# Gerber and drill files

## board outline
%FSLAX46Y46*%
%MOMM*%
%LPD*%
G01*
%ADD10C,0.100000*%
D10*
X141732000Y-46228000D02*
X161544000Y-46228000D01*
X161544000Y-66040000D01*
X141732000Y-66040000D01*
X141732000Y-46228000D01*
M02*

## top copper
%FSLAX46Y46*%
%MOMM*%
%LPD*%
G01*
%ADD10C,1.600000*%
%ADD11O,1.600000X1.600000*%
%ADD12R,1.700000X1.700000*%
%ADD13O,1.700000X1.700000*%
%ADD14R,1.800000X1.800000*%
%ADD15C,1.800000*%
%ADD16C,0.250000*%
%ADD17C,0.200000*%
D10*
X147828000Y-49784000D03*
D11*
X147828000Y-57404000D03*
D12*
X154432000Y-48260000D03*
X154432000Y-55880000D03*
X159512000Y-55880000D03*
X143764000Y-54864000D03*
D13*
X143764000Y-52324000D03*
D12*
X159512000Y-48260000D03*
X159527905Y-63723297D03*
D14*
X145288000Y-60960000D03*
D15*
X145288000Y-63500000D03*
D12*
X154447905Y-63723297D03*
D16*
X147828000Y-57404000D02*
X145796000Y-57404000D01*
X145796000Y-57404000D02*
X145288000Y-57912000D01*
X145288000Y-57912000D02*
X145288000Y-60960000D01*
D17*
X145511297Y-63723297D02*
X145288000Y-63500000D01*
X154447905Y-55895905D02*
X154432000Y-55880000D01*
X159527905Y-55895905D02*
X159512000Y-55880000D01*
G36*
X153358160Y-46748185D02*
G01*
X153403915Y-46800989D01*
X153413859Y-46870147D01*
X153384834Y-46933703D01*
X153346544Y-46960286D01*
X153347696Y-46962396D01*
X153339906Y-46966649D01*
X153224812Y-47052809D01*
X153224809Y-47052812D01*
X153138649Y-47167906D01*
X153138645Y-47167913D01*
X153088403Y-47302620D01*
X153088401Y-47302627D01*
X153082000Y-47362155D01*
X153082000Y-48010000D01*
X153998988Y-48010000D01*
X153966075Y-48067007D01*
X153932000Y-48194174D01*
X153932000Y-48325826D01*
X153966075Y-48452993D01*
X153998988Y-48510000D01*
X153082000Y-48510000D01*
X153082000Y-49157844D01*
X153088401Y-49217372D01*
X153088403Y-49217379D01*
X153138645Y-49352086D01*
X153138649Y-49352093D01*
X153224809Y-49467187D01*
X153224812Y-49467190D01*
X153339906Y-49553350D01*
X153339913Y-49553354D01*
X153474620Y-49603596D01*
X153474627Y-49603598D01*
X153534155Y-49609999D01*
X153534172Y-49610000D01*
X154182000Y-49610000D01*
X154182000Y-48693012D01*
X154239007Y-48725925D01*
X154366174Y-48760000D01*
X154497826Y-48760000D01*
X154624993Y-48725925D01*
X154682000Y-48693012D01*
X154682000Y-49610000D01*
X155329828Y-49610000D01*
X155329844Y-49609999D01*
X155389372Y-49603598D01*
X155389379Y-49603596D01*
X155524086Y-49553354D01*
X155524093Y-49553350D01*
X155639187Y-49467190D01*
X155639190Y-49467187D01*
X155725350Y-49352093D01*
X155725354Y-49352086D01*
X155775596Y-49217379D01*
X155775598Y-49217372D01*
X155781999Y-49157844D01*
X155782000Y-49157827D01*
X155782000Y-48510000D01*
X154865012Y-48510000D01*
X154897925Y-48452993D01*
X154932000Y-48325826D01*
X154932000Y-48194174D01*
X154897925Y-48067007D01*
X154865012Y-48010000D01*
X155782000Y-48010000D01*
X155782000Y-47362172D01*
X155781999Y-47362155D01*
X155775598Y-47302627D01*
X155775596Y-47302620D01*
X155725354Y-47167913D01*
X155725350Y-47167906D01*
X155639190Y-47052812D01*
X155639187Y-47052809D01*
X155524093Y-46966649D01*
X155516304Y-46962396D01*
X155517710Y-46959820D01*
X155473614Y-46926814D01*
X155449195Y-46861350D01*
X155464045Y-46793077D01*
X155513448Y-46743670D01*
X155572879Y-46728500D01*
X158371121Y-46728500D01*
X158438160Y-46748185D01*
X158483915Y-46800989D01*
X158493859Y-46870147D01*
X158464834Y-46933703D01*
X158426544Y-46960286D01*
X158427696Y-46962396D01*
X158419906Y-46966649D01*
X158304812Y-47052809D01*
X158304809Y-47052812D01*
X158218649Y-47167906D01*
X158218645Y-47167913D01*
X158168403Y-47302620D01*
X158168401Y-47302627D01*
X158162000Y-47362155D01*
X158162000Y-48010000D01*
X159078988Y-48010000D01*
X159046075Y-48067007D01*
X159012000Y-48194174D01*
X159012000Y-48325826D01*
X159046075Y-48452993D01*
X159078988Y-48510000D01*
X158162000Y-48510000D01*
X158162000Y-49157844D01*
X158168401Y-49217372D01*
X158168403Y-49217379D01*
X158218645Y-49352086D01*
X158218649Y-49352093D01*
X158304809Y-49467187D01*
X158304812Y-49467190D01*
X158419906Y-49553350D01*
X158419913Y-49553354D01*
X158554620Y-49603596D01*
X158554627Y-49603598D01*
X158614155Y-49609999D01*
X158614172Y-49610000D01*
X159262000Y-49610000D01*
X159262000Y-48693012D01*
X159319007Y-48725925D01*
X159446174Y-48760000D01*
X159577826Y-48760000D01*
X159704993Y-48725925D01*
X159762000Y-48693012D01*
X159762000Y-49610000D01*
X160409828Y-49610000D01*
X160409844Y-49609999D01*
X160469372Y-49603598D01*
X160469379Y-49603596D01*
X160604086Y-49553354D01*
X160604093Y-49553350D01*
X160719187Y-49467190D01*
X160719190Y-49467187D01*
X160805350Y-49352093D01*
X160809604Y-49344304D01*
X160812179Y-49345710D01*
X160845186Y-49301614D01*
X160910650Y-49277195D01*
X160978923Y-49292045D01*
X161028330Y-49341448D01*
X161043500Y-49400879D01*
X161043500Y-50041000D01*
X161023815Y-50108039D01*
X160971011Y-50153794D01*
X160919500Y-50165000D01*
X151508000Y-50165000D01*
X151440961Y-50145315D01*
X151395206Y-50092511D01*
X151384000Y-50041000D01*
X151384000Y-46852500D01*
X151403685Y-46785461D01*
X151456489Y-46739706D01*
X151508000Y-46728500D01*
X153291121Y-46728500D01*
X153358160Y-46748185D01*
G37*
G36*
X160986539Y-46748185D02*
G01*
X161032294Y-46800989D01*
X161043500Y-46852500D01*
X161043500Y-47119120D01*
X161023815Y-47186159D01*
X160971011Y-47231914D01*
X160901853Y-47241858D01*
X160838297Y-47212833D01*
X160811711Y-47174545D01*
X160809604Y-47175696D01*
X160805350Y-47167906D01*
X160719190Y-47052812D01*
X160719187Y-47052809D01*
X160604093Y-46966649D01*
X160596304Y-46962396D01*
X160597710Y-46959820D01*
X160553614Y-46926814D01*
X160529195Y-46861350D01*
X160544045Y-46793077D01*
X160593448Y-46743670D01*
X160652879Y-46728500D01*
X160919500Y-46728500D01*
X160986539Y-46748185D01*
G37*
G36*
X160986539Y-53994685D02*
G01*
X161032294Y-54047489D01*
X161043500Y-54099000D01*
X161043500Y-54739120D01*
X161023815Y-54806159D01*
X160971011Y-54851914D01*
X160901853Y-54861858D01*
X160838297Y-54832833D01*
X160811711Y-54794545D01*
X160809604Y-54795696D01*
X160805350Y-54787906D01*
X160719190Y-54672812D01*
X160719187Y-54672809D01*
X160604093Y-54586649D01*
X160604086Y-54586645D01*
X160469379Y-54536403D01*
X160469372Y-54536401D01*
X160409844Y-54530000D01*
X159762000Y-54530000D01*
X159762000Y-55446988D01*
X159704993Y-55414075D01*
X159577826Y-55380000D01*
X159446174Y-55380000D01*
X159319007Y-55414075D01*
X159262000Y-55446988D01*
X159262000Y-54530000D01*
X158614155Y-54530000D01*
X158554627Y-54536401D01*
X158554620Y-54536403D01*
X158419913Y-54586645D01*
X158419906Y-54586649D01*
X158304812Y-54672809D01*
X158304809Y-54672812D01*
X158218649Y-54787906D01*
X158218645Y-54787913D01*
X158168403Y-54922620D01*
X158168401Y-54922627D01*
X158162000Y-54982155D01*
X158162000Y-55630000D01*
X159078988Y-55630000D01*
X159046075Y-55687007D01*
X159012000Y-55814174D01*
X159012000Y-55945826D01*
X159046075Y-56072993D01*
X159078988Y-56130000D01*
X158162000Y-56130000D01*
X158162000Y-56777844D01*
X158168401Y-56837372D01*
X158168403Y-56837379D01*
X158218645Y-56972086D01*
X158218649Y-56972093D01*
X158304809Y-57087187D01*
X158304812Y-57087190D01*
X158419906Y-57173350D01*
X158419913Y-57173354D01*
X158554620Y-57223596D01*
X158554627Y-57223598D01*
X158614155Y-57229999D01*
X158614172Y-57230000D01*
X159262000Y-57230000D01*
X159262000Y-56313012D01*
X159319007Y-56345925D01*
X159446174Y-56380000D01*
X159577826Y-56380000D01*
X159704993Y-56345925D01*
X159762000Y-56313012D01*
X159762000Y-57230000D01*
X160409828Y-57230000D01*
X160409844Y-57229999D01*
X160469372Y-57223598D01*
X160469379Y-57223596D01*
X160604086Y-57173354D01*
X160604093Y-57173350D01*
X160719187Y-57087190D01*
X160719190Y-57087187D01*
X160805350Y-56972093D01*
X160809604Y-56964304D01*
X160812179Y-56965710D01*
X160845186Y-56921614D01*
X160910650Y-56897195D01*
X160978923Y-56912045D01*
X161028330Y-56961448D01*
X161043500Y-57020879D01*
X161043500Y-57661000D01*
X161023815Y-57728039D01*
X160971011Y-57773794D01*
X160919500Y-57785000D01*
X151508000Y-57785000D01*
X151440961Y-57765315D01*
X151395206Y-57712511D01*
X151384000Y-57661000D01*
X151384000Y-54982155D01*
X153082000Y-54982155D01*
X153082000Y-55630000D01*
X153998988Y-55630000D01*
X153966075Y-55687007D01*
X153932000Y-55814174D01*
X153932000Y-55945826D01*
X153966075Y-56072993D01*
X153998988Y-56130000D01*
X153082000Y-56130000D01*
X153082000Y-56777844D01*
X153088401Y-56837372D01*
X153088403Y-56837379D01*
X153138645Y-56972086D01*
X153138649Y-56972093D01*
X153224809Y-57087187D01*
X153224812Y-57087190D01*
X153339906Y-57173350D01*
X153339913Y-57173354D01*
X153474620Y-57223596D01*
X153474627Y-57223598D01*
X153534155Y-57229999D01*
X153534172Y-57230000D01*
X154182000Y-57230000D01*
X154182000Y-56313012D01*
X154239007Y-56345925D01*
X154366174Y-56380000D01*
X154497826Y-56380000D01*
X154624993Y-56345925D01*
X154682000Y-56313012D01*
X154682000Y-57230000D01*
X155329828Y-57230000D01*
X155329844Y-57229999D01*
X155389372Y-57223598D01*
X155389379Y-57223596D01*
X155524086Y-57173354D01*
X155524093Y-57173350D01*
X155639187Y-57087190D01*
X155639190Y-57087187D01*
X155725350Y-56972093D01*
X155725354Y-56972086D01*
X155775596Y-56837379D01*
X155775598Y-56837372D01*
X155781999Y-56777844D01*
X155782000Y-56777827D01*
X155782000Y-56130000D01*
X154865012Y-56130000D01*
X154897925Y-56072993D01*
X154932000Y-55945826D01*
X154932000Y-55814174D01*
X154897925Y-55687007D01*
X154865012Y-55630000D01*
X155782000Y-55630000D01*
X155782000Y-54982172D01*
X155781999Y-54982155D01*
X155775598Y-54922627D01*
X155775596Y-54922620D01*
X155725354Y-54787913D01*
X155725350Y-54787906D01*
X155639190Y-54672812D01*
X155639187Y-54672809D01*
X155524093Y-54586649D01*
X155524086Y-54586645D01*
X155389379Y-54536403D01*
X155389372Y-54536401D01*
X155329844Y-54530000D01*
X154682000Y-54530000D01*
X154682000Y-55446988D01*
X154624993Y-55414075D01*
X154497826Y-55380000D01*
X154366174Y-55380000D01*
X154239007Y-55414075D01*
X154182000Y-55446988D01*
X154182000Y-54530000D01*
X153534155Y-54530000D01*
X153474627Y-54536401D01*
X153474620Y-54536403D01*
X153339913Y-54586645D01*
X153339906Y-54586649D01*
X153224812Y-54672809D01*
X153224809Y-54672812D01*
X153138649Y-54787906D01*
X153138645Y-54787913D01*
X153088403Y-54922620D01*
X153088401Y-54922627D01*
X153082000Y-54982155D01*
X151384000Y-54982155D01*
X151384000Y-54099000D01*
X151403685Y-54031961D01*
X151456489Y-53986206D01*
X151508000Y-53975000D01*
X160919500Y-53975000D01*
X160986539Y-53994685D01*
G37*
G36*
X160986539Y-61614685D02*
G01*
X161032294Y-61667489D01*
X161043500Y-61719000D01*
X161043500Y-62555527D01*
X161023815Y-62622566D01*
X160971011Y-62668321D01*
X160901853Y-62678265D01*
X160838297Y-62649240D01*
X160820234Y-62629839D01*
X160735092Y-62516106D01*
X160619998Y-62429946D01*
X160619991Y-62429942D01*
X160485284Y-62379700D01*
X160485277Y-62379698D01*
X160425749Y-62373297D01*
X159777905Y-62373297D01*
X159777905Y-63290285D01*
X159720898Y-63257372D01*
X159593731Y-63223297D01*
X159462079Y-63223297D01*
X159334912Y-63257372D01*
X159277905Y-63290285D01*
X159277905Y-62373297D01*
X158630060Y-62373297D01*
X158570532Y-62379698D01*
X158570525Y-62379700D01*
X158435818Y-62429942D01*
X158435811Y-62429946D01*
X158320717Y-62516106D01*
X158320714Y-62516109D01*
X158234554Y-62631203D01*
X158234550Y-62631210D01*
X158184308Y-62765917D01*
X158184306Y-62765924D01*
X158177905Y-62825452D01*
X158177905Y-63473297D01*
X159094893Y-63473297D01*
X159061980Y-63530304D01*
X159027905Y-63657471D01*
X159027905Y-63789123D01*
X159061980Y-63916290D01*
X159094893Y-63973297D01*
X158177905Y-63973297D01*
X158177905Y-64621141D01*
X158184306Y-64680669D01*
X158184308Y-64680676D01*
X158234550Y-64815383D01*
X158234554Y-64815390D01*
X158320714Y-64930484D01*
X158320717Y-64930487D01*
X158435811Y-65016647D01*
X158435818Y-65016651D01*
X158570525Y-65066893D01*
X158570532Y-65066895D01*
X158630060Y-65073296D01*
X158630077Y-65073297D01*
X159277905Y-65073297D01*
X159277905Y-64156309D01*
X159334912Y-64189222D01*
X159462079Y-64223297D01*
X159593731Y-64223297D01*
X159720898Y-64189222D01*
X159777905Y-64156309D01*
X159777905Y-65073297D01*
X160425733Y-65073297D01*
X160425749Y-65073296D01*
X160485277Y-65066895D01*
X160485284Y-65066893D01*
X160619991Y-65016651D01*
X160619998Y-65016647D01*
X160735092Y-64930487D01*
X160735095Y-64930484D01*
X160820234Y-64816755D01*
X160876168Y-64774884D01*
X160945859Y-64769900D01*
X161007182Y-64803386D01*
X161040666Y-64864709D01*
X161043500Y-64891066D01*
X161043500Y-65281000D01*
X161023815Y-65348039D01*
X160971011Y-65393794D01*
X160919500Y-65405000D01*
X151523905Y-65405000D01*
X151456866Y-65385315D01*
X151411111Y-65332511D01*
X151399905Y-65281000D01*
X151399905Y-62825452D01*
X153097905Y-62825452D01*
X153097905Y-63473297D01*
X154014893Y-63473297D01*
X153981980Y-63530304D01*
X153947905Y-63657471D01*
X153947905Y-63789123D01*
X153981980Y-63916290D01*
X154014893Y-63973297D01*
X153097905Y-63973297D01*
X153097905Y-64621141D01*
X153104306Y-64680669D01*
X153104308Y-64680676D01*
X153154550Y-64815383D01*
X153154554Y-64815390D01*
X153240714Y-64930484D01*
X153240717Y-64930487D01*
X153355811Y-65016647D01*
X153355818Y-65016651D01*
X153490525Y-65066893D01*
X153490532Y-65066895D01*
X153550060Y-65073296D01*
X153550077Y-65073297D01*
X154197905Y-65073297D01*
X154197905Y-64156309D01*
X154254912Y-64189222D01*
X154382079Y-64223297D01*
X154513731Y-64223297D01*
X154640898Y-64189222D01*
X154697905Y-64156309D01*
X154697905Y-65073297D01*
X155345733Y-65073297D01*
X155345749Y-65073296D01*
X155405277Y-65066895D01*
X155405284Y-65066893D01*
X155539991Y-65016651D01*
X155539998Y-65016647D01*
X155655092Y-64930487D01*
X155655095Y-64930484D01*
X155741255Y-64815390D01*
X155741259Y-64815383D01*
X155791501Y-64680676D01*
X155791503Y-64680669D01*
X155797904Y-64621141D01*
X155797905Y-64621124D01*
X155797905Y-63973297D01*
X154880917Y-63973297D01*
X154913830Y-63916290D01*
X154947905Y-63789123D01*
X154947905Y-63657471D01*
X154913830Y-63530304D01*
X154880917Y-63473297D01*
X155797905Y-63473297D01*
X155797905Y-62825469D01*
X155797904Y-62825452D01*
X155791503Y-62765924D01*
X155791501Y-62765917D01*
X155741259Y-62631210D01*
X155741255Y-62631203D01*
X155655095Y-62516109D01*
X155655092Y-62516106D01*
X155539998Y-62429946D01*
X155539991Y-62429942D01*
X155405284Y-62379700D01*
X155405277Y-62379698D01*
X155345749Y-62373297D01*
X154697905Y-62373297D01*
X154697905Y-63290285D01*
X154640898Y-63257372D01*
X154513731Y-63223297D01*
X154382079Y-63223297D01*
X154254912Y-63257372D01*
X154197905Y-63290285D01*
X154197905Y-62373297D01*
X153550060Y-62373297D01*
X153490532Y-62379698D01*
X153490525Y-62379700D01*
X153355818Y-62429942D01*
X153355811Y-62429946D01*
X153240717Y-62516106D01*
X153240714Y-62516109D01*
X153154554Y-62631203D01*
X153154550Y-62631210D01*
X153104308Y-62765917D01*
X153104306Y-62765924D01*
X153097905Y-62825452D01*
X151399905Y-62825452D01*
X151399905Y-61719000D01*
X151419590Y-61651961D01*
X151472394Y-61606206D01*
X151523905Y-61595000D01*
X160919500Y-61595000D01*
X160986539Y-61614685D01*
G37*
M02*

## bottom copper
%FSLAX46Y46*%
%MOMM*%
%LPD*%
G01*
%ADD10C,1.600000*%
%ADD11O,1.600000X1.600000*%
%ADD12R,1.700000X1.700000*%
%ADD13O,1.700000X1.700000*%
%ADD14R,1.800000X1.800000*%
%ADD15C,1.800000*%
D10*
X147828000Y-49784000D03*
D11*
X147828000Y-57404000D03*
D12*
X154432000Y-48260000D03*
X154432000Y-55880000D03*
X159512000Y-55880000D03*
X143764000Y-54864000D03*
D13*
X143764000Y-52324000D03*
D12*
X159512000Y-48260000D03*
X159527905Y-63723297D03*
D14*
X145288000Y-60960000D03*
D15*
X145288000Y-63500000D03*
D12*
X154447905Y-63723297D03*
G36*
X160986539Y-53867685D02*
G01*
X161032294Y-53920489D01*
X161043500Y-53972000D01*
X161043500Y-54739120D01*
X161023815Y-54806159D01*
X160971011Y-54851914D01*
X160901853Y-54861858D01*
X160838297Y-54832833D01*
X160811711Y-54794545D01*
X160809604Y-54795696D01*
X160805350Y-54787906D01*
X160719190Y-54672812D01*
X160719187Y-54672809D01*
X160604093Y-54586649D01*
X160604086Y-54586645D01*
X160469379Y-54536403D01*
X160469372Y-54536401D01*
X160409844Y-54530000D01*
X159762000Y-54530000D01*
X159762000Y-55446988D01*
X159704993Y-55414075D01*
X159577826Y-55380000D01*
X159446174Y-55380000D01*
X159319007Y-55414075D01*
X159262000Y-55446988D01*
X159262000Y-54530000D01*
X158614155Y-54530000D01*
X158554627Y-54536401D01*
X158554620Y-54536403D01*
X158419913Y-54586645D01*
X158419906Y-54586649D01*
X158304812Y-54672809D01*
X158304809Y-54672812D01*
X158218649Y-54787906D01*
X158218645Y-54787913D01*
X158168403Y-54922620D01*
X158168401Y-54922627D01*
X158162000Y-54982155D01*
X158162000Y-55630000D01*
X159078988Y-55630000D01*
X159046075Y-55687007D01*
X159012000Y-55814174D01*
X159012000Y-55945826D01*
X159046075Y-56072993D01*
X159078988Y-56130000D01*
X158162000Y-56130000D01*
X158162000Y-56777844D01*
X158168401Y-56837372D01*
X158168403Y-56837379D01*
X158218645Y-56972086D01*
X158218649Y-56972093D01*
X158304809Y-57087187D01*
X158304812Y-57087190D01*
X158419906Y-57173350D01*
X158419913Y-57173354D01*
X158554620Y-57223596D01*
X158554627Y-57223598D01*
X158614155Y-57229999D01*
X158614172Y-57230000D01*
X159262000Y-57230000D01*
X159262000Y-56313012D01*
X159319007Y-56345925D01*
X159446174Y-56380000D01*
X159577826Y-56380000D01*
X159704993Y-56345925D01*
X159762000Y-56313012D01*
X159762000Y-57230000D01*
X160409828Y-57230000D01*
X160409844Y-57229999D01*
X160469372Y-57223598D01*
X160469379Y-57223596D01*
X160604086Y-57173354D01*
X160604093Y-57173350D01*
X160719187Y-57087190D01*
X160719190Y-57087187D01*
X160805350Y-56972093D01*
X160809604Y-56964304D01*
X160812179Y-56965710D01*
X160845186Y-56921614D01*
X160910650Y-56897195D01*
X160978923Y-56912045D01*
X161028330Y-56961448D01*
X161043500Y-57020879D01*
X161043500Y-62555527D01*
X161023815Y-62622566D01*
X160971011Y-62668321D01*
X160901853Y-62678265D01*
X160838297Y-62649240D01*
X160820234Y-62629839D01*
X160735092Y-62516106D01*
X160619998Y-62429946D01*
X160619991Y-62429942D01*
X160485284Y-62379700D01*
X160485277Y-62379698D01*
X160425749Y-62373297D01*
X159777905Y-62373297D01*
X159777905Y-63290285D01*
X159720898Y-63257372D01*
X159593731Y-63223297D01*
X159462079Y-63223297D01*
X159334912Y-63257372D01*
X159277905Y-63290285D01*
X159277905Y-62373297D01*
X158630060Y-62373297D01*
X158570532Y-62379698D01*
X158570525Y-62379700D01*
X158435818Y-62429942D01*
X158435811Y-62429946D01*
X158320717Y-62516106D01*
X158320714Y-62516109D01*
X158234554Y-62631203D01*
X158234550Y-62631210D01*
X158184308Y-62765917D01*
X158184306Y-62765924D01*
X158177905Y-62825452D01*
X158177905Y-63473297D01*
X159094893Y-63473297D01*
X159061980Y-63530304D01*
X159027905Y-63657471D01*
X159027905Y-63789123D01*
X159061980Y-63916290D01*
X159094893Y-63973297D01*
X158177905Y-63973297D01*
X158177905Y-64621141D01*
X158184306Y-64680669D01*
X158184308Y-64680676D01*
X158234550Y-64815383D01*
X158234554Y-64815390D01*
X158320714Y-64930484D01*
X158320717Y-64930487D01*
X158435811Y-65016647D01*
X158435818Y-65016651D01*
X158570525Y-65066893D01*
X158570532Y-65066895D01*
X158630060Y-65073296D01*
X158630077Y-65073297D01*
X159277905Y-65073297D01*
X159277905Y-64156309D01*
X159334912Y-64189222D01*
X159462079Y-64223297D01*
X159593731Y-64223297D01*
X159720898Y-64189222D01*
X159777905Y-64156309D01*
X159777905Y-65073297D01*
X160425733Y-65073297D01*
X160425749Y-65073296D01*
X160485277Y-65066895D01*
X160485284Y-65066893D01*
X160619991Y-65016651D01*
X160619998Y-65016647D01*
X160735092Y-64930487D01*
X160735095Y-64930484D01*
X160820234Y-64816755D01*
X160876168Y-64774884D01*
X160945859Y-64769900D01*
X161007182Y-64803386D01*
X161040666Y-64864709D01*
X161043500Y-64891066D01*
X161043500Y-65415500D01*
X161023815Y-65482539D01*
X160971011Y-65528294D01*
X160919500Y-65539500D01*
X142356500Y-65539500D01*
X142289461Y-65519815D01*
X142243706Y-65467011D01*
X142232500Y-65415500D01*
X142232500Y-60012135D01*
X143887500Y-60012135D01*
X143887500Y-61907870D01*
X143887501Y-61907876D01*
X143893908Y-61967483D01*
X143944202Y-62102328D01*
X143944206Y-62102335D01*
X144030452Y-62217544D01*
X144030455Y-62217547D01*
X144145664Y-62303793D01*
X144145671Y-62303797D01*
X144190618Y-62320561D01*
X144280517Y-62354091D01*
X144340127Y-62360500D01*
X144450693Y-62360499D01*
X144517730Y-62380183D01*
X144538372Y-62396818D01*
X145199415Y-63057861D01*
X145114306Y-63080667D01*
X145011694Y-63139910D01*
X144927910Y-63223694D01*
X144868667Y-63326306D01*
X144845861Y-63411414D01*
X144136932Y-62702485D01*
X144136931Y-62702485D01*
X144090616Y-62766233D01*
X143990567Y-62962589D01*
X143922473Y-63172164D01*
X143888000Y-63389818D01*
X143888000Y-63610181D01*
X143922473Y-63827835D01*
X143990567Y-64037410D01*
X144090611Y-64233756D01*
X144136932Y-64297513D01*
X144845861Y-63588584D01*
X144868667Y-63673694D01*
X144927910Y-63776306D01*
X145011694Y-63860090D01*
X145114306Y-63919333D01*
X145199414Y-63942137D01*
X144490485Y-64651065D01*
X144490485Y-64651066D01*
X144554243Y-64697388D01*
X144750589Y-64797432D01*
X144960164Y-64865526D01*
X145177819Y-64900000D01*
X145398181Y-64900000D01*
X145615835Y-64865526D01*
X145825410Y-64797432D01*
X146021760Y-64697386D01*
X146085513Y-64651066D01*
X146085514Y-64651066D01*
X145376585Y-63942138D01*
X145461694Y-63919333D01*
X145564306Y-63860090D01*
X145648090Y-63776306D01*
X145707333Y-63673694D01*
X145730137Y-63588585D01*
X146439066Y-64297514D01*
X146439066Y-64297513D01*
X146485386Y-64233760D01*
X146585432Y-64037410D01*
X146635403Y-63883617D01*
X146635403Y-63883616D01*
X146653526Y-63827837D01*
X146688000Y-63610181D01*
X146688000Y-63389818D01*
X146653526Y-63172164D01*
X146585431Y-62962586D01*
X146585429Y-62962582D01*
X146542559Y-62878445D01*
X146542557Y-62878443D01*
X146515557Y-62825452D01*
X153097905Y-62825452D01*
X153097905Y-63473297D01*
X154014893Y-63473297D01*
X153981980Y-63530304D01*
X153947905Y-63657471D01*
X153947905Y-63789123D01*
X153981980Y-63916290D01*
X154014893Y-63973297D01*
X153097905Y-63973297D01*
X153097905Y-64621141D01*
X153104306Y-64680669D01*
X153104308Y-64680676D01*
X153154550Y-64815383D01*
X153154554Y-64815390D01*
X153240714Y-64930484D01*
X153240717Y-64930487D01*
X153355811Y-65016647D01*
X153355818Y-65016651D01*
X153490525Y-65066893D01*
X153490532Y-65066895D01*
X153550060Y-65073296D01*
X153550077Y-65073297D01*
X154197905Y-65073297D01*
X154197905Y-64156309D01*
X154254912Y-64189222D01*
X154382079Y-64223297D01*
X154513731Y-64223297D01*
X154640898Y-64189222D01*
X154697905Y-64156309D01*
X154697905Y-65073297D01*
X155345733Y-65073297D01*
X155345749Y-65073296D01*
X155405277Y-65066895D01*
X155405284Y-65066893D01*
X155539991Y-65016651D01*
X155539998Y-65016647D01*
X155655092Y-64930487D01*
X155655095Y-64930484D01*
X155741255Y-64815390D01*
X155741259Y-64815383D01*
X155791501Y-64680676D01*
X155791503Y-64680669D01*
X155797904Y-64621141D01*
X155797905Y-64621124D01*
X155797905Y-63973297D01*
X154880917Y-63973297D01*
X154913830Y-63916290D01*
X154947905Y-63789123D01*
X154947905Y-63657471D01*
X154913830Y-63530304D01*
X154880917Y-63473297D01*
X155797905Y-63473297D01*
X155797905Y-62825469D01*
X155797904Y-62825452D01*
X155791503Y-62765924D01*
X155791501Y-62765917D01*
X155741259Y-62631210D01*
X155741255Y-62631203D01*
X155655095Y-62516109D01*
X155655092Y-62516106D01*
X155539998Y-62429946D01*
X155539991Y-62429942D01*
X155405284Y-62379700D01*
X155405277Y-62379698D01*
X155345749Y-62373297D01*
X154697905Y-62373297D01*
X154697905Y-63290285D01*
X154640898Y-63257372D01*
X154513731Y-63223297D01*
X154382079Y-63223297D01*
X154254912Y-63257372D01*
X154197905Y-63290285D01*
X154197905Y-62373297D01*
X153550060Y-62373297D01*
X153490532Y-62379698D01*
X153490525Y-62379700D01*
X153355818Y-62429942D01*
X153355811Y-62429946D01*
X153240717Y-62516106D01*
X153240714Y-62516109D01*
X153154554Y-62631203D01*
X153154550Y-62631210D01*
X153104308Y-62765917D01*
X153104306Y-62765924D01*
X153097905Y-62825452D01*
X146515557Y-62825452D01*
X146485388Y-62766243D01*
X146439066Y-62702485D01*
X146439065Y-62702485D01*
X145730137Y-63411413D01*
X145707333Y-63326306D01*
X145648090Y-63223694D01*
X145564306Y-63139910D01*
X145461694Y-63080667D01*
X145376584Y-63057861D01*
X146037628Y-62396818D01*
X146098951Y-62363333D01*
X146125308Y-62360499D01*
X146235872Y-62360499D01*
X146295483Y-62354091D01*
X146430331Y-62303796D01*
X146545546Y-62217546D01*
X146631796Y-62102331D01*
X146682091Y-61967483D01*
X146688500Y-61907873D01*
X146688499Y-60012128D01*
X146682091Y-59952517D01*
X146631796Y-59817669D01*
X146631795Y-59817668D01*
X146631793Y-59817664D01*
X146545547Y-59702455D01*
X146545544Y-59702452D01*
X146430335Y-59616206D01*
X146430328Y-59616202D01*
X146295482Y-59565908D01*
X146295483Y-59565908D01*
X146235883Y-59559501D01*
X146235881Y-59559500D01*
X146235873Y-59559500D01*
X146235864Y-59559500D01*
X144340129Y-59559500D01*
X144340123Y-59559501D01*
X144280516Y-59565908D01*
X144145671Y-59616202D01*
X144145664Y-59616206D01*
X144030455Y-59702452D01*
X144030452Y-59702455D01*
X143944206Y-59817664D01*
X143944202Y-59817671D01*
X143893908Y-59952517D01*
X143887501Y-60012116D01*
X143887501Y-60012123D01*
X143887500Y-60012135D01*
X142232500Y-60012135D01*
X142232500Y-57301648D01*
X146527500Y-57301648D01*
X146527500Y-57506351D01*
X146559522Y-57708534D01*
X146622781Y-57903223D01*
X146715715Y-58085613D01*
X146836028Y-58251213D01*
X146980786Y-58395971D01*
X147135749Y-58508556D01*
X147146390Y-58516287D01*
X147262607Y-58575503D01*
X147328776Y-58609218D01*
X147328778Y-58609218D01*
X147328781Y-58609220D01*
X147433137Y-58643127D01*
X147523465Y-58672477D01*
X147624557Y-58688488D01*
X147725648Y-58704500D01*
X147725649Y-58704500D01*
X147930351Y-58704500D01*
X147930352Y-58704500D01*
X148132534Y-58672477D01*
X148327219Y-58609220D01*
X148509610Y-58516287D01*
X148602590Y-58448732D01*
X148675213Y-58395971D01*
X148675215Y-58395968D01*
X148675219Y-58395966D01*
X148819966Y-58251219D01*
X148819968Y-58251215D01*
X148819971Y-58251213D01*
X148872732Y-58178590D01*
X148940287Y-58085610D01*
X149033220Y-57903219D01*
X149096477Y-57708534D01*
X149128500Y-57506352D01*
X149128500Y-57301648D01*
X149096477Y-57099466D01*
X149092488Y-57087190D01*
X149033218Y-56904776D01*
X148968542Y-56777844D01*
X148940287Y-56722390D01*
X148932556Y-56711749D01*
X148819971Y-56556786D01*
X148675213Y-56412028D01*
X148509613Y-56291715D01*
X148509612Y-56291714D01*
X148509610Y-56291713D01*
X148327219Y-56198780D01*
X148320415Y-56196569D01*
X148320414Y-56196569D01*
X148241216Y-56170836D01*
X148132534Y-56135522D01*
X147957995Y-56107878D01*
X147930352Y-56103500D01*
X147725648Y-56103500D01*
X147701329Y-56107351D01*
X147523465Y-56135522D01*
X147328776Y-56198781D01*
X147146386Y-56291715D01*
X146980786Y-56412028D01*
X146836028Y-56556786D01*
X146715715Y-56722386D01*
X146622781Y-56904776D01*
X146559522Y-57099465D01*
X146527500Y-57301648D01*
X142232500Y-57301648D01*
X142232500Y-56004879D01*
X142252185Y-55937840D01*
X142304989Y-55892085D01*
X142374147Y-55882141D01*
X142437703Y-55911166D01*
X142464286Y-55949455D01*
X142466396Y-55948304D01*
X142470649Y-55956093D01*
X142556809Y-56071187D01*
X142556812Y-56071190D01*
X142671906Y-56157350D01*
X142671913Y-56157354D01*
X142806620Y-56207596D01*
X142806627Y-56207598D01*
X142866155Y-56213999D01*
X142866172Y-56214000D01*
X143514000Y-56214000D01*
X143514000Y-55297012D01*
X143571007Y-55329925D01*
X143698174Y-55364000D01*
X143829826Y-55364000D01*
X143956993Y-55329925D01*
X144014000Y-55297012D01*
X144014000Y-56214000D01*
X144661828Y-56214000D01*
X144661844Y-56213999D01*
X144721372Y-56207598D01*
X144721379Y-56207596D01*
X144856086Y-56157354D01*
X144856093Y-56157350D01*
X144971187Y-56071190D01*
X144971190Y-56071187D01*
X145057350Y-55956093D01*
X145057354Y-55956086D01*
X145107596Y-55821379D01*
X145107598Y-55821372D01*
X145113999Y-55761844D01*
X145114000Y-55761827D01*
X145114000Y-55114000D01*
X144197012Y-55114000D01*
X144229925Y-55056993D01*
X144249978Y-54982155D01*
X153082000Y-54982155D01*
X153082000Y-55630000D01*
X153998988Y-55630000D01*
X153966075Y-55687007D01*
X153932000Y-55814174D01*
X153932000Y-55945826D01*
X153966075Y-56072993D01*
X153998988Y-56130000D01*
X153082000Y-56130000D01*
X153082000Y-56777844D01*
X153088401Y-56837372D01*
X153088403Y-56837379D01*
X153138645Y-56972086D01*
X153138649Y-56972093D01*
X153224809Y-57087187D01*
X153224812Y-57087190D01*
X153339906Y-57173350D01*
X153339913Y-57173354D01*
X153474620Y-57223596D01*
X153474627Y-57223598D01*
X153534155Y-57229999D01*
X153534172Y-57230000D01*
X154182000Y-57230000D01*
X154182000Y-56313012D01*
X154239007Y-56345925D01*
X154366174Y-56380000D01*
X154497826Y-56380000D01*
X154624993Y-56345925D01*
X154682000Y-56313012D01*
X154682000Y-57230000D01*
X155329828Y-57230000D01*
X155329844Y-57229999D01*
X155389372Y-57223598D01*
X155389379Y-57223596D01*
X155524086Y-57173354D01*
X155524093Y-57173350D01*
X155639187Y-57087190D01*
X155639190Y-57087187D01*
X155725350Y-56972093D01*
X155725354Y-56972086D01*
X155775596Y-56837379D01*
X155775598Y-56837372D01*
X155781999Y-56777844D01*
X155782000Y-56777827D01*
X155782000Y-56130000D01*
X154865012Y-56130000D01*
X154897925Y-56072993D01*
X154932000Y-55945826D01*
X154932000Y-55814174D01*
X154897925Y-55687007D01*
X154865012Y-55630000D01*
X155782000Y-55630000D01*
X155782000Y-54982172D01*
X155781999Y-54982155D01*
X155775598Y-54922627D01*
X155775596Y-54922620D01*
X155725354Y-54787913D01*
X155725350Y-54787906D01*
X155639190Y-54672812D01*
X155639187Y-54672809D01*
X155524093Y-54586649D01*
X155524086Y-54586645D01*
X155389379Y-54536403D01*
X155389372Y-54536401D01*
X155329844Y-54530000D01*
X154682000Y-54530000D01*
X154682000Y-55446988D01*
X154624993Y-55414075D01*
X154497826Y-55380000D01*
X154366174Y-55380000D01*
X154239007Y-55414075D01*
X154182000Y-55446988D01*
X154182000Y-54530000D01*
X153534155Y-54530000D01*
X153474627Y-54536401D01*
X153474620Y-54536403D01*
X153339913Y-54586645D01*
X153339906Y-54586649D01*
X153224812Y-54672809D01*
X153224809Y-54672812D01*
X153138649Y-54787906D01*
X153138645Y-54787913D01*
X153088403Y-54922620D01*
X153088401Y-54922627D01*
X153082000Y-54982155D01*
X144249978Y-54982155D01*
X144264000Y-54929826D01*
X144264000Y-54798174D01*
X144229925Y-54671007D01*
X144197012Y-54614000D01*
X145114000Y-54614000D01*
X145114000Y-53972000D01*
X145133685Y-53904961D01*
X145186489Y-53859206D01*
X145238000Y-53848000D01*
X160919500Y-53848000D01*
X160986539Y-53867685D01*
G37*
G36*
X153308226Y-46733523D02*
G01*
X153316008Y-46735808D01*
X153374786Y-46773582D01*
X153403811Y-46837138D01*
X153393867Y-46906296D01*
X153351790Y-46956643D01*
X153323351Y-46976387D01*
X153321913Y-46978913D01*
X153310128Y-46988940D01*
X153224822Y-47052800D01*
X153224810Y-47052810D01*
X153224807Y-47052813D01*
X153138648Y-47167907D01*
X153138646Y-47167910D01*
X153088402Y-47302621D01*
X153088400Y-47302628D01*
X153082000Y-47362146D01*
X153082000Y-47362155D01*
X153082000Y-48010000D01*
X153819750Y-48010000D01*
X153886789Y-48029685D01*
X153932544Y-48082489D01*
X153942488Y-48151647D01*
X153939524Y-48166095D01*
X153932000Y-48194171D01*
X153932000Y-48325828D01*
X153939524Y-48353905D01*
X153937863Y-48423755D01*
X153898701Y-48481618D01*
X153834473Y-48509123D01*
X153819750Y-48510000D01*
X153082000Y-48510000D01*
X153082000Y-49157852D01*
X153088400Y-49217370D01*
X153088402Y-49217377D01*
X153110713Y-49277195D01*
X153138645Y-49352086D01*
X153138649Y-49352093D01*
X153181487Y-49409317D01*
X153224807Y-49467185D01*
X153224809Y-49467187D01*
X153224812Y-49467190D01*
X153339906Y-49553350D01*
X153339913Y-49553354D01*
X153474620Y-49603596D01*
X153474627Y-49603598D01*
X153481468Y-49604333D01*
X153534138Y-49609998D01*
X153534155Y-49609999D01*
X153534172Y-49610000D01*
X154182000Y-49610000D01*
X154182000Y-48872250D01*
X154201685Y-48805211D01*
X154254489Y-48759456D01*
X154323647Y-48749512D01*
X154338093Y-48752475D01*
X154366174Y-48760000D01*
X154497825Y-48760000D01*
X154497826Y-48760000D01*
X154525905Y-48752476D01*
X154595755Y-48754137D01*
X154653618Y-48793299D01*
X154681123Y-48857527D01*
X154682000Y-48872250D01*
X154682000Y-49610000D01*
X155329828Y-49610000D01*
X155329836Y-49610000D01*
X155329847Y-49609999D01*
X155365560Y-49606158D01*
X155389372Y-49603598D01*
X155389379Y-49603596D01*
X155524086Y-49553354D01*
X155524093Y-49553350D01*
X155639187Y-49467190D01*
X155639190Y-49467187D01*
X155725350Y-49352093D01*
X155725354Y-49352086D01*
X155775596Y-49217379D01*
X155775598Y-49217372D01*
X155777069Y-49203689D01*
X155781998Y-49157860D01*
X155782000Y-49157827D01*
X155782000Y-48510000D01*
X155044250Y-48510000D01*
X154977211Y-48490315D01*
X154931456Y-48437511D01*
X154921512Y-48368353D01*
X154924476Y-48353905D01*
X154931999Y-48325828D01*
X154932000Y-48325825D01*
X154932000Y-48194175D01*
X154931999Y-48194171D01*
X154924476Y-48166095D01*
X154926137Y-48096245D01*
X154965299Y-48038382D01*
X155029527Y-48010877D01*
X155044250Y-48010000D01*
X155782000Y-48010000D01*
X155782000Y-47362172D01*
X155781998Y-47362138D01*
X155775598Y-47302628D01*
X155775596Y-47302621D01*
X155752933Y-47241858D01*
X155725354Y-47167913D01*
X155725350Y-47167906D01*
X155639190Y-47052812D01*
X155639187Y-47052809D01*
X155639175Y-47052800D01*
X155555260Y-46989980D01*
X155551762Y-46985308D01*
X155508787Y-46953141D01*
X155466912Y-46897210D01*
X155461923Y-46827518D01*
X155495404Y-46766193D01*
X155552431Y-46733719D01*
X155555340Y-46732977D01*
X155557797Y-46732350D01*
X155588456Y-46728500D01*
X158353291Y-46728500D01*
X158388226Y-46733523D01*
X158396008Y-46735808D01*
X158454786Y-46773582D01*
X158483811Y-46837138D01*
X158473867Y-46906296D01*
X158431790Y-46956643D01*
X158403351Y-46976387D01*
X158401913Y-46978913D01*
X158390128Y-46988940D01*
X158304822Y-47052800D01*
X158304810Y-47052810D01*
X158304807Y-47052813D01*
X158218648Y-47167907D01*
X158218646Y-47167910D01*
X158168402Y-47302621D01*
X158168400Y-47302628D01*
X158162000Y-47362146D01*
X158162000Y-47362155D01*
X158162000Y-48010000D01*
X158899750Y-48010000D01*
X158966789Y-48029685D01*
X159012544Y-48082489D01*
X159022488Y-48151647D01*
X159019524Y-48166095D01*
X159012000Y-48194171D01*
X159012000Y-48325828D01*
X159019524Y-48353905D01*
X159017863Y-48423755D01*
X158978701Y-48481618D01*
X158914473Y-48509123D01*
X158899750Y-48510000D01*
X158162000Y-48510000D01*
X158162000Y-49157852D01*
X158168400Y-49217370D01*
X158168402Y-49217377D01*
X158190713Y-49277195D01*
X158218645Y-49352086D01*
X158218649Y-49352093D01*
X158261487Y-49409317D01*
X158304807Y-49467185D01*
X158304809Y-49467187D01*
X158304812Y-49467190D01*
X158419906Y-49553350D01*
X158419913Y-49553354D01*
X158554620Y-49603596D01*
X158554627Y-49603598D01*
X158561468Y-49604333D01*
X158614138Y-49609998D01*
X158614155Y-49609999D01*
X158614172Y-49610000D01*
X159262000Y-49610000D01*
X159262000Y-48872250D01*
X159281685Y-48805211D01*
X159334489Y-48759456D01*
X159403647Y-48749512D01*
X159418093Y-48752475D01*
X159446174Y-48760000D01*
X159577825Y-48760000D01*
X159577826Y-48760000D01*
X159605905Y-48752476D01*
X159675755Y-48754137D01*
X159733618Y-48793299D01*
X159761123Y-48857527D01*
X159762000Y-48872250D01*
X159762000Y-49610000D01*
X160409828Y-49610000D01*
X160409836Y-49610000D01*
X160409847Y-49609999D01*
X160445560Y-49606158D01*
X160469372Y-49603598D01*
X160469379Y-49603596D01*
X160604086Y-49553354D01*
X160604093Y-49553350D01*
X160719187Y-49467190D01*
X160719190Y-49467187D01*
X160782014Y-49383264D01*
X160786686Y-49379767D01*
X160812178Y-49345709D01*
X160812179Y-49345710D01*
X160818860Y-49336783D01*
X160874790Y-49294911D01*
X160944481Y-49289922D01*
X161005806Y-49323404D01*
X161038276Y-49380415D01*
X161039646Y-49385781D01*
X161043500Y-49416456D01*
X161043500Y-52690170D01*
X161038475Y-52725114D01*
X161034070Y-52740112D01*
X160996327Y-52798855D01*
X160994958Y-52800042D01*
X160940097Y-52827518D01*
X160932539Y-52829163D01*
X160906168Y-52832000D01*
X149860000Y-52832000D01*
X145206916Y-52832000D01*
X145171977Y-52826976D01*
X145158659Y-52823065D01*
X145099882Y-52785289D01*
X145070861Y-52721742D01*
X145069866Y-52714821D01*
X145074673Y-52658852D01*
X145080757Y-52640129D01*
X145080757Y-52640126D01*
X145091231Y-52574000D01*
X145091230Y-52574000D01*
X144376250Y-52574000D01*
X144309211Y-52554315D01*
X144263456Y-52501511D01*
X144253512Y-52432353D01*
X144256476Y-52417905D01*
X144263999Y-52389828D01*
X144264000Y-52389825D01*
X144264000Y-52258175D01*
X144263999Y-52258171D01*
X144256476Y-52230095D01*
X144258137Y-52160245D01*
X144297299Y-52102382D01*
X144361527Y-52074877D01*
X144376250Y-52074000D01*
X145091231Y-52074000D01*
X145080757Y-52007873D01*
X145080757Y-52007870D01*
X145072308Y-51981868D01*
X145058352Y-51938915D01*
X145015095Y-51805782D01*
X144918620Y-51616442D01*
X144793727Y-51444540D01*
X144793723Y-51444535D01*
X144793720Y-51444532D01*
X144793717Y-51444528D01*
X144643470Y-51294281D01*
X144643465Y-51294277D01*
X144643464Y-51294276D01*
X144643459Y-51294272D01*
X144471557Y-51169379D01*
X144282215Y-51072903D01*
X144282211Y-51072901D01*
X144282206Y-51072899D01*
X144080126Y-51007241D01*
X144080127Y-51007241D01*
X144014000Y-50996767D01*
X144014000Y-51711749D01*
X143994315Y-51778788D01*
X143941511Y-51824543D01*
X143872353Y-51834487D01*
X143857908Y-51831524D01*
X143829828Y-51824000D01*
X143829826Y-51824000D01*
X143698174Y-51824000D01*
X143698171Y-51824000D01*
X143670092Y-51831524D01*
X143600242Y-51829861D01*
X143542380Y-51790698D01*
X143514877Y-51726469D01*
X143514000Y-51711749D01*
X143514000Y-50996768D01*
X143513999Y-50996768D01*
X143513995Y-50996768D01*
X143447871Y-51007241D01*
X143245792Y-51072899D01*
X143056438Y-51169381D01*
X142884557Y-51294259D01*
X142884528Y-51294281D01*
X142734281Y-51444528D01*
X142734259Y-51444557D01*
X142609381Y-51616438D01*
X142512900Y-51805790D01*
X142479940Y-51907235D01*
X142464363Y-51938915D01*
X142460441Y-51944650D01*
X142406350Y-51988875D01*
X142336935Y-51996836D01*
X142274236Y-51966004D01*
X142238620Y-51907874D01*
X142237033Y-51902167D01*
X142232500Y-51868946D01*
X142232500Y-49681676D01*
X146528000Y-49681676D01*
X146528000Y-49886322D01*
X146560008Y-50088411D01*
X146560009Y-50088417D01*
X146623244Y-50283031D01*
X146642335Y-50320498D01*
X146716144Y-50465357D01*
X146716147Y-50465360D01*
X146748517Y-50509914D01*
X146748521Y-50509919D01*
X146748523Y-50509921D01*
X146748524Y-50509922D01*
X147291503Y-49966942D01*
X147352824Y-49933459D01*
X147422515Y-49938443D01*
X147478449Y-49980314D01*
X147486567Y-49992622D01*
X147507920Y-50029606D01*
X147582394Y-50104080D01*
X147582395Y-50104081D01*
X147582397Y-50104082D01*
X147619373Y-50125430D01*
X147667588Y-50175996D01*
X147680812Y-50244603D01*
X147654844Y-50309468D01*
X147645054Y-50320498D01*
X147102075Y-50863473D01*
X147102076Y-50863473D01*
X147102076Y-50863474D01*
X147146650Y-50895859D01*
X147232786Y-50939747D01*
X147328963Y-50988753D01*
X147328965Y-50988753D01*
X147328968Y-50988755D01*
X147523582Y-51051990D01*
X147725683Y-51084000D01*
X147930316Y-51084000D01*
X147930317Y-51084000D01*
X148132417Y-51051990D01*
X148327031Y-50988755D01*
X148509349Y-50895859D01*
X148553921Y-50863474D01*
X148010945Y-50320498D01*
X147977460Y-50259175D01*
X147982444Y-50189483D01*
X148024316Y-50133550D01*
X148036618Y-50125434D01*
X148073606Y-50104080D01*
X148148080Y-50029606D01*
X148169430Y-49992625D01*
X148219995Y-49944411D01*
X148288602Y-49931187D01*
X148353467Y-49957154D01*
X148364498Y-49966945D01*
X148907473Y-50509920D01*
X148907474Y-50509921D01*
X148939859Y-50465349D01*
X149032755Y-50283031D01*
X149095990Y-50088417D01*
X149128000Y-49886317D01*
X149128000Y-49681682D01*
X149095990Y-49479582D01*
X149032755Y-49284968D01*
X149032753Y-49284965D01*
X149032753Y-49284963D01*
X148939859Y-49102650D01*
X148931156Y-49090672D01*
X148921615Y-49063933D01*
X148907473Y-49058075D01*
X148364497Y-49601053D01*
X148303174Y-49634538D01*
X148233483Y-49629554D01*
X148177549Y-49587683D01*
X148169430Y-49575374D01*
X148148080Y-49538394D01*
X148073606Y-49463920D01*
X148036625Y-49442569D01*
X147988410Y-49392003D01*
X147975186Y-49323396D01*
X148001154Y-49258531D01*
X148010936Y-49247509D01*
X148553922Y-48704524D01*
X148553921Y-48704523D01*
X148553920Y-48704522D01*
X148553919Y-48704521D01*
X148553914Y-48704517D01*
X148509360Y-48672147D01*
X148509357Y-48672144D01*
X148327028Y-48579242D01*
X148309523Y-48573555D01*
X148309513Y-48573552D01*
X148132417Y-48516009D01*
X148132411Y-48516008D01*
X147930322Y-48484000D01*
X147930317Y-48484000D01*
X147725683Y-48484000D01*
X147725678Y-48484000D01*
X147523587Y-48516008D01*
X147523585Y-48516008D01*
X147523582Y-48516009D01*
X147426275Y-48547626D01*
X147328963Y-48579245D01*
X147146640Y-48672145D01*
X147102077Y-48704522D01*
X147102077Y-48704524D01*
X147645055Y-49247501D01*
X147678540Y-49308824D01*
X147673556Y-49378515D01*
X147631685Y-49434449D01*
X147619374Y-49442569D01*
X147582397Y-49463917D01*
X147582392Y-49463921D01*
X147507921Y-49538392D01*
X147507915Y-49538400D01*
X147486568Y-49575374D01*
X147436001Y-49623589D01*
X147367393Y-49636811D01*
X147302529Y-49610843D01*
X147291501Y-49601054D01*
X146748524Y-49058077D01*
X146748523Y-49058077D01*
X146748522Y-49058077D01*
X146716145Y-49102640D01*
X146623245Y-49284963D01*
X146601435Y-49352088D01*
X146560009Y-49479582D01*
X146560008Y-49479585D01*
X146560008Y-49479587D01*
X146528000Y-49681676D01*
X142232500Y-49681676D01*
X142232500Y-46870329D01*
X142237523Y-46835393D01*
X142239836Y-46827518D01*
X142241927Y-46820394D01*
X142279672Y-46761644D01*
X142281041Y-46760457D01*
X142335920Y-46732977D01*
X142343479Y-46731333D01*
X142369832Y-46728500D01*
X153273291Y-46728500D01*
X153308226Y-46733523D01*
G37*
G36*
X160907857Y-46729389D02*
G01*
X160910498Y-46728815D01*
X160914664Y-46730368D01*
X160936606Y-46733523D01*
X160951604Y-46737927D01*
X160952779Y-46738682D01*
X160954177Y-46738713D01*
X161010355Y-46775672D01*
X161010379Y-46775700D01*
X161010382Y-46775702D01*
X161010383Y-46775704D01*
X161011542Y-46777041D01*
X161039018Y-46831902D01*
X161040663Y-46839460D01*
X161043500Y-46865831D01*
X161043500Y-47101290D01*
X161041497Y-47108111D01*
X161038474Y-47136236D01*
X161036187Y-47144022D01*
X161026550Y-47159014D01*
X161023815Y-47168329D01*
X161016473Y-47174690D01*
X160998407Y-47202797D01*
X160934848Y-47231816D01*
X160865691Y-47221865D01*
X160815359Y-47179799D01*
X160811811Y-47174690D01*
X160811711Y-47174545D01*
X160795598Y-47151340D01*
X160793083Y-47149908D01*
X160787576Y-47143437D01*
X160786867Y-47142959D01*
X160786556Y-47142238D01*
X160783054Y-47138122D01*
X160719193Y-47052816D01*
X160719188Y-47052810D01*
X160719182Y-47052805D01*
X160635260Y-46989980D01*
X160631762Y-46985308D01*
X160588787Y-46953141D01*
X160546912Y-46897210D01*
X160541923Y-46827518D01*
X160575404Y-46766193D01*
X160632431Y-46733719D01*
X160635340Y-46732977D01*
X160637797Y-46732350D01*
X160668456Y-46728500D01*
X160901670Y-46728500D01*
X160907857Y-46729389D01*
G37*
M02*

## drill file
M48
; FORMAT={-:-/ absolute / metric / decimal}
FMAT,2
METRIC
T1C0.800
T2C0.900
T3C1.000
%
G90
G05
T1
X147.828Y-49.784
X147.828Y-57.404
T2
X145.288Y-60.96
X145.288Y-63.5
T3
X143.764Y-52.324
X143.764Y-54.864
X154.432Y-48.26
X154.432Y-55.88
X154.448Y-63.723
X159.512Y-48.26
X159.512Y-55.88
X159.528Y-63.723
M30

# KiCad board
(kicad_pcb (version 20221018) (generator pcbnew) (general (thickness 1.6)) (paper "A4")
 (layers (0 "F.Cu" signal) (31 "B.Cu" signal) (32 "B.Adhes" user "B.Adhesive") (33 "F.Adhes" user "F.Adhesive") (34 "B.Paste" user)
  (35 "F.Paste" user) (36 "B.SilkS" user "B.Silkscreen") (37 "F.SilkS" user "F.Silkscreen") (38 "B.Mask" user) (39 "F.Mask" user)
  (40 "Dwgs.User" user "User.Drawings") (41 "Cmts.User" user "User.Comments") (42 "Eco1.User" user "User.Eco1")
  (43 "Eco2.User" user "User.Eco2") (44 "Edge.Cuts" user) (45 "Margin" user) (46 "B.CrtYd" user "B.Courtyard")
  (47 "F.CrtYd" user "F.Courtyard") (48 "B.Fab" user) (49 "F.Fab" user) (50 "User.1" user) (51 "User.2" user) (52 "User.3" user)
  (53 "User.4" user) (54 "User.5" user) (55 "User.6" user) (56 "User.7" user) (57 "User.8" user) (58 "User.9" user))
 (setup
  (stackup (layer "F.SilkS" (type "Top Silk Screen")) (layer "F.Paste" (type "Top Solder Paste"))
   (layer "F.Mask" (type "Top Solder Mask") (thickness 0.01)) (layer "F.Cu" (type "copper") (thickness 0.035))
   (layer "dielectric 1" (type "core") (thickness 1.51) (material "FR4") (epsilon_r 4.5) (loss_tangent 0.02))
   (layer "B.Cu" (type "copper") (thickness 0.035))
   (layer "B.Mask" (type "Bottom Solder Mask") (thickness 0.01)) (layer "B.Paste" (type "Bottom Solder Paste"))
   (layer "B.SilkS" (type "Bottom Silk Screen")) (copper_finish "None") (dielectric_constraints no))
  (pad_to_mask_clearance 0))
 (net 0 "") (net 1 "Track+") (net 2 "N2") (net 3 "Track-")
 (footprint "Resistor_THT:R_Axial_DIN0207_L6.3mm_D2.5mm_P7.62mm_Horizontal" (layer "F.Cu") (at 147.828 49.784 -90)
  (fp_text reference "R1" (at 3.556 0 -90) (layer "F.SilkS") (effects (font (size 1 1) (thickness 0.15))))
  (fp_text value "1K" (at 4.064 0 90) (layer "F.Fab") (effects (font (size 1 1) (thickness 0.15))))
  (pad "1" thru_hole circle (at 0 0 270) (size 1.6 1.6) (drill 0.8) (layers "*.Cu" "*.Mask") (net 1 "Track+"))
  (pad "2" thru_hole oval (at 7.62 0 270) (size 1.6 1.6) (drill 0.8) (layers "*.Cu" "*.Mask") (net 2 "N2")))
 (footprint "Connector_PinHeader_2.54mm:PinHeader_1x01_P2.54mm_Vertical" (layer "F.Cu") (at 154.432 48.26)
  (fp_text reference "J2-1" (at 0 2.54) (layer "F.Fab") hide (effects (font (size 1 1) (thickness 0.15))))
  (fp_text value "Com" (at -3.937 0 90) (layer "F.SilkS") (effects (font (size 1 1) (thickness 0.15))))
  (pad "1" thru_hole rect (at 0 0) (size 1.7 1.7) (drill 1) (layers "*.Cu" "*.Mask") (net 1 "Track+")))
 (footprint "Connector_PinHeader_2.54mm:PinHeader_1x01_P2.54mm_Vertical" (layer "F.Cu") (at 154.432 55.88)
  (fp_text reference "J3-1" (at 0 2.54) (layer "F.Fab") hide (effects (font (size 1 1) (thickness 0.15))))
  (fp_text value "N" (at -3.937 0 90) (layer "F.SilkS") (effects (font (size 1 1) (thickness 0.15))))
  (pad "1" thru_hole rect (at 0 0) (size 1.7 1.7) (drill 1) (layers "*.Cu" "*.Mask") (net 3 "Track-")))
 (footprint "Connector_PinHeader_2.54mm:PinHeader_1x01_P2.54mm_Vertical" (layer "F.Cu") (at 159.512 55.88)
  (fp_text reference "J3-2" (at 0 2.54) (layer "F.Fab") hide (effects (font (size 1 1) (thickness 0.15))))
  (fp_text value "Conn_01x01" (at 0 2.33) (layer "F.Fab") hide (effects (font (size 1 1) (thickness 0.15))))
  (pad "1" thru_hole rect (at 0 0) (size 1.7 1.7) (drill 1) (layers "*.Cu" "*.Mask") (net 3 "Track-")))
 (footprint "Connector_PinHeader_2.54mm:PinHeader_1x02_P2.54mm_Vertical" (layer "F.Cu") (at 143.764 54.864 180)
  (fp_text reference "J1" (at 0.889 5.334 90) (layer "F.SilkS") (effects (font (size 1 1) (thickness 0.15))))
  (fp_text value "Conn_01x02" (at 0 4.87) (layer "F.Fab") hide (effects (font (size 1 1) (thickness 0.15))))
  (pad "1" thru_hole rect (at 0 0 180) (size 1.7 1.7) (drill 1) (layers "*.Cu" "*.Mask") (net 3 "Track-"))
  (pad "2" thru_hole oval (at 0 2.54 180) (size 1.7 1.7) (drill 1) (layers "*.Cu" "*.Mask") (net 1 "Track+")))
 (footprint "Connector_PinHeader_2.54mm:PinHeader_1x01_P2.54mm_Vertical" (layer "F.Cu") (at 159.512 48.26)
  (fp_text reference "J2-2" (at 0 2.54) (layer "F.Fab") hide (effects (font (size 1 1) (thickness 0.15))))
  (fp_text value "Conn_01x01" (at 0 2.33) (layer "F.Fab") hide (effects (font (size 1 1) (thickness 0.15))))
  (pad "1" thru_hole rect (at 0 0) (size 1.7 1.7) (drill 1) (layers "*.Cu" "*.Mask") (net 1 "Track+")))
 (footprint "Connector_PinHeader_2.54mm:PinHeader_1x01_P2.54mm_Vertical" (layer "F.Cu") (at 159.527905 63.723297)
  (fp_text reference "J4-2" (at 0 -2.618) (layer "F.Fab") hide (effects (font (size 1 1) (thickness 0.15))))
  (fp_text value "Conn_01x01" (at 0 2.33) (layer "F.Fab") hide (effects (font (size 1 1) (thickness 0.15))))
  (pad "1" thru_hole rect (at 0 0) (size 1.7 1.7) (drill 1) (layers "*.Cu" "*.Mask") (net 3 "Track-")))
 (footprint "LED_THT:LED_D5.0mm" (layer "F.Cu") (at 145.288 60.96 -90)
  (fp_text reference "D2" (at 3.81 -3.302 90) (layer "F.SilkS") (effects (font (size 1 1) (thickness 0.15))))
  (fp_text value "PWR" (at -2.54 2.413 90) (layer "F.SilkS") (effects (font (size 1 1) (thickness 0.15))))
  (pad "1" thru_hole rect (at 0 0 270) (size 1.8 1.8) (drill 0.9) (layers "*.Cu" "*.Mask") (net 2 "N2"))
  (pad "2" thru_hole circle (at 2.54 0 270) (size 1.8 1.8) (drill 0.9) (layers "*.Cu" "*.Mask") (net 3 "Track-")))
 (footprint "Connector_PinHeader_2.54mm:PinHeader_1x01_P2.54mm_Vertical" (layer "F.Cu") (at 154.447905 63.723297)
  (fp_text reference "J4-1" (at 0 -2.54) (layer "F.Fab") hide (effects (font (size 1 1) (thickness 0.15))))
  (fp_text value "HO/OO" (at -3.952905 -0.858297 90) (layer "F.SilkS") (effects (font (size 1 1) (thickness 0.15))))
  (pad "1" thru_hole rect (at 0 0) (size 1.7 1.7) (drill 1) (layers "*.Cu" "*.Mask") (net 3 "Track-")))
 (gr_poly
  (pts (xy 141.732 46.228) (xy 161.544 46.228) (xy 161.544 66.04) (xy 141.732 66.04)) (stroke (width 0.1) (type solid)) (fill none)
  (layer "Edge.Cuts"))
 (segment (start 147.828 57.404) (end 145.796 57.404) (width 0.25) (layer "F.Cu") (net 2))
 (segment (start 145.796 57.404) (end 145.288 57.912) (width 0.25) (layer "F.Cu") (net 2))
 (segment (start 145.288 57.912) (end 145.288 60.96) (width 0.25) (layer "F.Cu") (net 2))
 (segment (start 145.511297 63.723297) (end 145.288 63.5) (width 0.2) (layer "F.Cu") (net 3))
 (segment (start 154.447905 55.895905) (end 154.432 55.88) (width 0.2) (layer "F.Cu") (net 3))
 (segment (start 159.527905 55.895905) (end 159.512 55.88) (width 0.2) (layer "F.Cu") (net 3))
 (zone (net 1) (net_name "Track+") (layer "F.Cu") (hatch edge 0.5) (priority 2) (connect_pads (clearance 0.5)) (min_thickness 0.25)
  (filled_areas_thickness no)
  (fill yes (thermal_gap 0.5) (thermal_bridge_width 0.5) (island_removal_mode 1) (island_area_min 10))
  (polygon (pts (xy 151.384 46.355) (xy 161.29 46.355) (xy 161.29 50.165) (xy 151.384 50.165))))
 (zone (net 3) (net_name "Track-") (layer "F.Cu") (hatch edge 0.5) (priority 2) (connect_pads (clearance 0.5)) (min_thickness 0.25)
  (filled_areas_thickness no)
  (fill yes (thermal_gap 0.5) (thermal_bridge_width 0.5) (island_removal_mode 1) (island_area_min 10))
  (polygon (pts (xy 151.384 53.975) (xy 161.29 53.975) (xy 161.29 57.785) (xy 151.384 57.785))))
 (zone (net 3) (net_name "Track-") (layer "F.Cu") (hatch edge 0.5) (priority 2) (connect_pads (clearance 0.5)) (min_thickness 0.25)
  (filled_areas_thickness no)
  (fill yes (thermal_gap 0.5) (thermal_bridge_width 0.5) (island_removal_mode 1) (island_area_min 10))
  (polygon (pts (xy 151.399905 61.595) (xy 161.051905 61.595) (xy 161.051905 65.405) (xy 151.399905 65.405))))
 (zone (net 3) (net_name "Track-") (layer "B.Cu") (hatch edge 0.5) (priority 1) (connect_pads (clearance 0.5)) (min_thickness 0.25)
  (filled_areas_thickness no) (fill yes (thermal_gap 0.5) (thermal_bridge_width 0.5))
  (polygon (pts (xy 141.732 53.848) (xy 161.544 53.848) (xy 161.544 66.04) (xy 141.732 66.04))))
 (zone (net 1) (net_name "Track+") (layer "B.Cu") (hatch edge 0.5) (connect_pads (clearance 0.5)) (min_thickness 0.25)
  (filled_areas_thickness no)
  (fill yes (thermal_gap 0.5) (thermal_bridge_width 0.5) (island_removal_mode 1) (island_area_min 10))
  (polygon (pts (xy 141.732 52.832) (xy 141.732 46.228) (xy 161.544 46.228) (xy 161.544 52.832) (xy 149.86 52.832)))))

